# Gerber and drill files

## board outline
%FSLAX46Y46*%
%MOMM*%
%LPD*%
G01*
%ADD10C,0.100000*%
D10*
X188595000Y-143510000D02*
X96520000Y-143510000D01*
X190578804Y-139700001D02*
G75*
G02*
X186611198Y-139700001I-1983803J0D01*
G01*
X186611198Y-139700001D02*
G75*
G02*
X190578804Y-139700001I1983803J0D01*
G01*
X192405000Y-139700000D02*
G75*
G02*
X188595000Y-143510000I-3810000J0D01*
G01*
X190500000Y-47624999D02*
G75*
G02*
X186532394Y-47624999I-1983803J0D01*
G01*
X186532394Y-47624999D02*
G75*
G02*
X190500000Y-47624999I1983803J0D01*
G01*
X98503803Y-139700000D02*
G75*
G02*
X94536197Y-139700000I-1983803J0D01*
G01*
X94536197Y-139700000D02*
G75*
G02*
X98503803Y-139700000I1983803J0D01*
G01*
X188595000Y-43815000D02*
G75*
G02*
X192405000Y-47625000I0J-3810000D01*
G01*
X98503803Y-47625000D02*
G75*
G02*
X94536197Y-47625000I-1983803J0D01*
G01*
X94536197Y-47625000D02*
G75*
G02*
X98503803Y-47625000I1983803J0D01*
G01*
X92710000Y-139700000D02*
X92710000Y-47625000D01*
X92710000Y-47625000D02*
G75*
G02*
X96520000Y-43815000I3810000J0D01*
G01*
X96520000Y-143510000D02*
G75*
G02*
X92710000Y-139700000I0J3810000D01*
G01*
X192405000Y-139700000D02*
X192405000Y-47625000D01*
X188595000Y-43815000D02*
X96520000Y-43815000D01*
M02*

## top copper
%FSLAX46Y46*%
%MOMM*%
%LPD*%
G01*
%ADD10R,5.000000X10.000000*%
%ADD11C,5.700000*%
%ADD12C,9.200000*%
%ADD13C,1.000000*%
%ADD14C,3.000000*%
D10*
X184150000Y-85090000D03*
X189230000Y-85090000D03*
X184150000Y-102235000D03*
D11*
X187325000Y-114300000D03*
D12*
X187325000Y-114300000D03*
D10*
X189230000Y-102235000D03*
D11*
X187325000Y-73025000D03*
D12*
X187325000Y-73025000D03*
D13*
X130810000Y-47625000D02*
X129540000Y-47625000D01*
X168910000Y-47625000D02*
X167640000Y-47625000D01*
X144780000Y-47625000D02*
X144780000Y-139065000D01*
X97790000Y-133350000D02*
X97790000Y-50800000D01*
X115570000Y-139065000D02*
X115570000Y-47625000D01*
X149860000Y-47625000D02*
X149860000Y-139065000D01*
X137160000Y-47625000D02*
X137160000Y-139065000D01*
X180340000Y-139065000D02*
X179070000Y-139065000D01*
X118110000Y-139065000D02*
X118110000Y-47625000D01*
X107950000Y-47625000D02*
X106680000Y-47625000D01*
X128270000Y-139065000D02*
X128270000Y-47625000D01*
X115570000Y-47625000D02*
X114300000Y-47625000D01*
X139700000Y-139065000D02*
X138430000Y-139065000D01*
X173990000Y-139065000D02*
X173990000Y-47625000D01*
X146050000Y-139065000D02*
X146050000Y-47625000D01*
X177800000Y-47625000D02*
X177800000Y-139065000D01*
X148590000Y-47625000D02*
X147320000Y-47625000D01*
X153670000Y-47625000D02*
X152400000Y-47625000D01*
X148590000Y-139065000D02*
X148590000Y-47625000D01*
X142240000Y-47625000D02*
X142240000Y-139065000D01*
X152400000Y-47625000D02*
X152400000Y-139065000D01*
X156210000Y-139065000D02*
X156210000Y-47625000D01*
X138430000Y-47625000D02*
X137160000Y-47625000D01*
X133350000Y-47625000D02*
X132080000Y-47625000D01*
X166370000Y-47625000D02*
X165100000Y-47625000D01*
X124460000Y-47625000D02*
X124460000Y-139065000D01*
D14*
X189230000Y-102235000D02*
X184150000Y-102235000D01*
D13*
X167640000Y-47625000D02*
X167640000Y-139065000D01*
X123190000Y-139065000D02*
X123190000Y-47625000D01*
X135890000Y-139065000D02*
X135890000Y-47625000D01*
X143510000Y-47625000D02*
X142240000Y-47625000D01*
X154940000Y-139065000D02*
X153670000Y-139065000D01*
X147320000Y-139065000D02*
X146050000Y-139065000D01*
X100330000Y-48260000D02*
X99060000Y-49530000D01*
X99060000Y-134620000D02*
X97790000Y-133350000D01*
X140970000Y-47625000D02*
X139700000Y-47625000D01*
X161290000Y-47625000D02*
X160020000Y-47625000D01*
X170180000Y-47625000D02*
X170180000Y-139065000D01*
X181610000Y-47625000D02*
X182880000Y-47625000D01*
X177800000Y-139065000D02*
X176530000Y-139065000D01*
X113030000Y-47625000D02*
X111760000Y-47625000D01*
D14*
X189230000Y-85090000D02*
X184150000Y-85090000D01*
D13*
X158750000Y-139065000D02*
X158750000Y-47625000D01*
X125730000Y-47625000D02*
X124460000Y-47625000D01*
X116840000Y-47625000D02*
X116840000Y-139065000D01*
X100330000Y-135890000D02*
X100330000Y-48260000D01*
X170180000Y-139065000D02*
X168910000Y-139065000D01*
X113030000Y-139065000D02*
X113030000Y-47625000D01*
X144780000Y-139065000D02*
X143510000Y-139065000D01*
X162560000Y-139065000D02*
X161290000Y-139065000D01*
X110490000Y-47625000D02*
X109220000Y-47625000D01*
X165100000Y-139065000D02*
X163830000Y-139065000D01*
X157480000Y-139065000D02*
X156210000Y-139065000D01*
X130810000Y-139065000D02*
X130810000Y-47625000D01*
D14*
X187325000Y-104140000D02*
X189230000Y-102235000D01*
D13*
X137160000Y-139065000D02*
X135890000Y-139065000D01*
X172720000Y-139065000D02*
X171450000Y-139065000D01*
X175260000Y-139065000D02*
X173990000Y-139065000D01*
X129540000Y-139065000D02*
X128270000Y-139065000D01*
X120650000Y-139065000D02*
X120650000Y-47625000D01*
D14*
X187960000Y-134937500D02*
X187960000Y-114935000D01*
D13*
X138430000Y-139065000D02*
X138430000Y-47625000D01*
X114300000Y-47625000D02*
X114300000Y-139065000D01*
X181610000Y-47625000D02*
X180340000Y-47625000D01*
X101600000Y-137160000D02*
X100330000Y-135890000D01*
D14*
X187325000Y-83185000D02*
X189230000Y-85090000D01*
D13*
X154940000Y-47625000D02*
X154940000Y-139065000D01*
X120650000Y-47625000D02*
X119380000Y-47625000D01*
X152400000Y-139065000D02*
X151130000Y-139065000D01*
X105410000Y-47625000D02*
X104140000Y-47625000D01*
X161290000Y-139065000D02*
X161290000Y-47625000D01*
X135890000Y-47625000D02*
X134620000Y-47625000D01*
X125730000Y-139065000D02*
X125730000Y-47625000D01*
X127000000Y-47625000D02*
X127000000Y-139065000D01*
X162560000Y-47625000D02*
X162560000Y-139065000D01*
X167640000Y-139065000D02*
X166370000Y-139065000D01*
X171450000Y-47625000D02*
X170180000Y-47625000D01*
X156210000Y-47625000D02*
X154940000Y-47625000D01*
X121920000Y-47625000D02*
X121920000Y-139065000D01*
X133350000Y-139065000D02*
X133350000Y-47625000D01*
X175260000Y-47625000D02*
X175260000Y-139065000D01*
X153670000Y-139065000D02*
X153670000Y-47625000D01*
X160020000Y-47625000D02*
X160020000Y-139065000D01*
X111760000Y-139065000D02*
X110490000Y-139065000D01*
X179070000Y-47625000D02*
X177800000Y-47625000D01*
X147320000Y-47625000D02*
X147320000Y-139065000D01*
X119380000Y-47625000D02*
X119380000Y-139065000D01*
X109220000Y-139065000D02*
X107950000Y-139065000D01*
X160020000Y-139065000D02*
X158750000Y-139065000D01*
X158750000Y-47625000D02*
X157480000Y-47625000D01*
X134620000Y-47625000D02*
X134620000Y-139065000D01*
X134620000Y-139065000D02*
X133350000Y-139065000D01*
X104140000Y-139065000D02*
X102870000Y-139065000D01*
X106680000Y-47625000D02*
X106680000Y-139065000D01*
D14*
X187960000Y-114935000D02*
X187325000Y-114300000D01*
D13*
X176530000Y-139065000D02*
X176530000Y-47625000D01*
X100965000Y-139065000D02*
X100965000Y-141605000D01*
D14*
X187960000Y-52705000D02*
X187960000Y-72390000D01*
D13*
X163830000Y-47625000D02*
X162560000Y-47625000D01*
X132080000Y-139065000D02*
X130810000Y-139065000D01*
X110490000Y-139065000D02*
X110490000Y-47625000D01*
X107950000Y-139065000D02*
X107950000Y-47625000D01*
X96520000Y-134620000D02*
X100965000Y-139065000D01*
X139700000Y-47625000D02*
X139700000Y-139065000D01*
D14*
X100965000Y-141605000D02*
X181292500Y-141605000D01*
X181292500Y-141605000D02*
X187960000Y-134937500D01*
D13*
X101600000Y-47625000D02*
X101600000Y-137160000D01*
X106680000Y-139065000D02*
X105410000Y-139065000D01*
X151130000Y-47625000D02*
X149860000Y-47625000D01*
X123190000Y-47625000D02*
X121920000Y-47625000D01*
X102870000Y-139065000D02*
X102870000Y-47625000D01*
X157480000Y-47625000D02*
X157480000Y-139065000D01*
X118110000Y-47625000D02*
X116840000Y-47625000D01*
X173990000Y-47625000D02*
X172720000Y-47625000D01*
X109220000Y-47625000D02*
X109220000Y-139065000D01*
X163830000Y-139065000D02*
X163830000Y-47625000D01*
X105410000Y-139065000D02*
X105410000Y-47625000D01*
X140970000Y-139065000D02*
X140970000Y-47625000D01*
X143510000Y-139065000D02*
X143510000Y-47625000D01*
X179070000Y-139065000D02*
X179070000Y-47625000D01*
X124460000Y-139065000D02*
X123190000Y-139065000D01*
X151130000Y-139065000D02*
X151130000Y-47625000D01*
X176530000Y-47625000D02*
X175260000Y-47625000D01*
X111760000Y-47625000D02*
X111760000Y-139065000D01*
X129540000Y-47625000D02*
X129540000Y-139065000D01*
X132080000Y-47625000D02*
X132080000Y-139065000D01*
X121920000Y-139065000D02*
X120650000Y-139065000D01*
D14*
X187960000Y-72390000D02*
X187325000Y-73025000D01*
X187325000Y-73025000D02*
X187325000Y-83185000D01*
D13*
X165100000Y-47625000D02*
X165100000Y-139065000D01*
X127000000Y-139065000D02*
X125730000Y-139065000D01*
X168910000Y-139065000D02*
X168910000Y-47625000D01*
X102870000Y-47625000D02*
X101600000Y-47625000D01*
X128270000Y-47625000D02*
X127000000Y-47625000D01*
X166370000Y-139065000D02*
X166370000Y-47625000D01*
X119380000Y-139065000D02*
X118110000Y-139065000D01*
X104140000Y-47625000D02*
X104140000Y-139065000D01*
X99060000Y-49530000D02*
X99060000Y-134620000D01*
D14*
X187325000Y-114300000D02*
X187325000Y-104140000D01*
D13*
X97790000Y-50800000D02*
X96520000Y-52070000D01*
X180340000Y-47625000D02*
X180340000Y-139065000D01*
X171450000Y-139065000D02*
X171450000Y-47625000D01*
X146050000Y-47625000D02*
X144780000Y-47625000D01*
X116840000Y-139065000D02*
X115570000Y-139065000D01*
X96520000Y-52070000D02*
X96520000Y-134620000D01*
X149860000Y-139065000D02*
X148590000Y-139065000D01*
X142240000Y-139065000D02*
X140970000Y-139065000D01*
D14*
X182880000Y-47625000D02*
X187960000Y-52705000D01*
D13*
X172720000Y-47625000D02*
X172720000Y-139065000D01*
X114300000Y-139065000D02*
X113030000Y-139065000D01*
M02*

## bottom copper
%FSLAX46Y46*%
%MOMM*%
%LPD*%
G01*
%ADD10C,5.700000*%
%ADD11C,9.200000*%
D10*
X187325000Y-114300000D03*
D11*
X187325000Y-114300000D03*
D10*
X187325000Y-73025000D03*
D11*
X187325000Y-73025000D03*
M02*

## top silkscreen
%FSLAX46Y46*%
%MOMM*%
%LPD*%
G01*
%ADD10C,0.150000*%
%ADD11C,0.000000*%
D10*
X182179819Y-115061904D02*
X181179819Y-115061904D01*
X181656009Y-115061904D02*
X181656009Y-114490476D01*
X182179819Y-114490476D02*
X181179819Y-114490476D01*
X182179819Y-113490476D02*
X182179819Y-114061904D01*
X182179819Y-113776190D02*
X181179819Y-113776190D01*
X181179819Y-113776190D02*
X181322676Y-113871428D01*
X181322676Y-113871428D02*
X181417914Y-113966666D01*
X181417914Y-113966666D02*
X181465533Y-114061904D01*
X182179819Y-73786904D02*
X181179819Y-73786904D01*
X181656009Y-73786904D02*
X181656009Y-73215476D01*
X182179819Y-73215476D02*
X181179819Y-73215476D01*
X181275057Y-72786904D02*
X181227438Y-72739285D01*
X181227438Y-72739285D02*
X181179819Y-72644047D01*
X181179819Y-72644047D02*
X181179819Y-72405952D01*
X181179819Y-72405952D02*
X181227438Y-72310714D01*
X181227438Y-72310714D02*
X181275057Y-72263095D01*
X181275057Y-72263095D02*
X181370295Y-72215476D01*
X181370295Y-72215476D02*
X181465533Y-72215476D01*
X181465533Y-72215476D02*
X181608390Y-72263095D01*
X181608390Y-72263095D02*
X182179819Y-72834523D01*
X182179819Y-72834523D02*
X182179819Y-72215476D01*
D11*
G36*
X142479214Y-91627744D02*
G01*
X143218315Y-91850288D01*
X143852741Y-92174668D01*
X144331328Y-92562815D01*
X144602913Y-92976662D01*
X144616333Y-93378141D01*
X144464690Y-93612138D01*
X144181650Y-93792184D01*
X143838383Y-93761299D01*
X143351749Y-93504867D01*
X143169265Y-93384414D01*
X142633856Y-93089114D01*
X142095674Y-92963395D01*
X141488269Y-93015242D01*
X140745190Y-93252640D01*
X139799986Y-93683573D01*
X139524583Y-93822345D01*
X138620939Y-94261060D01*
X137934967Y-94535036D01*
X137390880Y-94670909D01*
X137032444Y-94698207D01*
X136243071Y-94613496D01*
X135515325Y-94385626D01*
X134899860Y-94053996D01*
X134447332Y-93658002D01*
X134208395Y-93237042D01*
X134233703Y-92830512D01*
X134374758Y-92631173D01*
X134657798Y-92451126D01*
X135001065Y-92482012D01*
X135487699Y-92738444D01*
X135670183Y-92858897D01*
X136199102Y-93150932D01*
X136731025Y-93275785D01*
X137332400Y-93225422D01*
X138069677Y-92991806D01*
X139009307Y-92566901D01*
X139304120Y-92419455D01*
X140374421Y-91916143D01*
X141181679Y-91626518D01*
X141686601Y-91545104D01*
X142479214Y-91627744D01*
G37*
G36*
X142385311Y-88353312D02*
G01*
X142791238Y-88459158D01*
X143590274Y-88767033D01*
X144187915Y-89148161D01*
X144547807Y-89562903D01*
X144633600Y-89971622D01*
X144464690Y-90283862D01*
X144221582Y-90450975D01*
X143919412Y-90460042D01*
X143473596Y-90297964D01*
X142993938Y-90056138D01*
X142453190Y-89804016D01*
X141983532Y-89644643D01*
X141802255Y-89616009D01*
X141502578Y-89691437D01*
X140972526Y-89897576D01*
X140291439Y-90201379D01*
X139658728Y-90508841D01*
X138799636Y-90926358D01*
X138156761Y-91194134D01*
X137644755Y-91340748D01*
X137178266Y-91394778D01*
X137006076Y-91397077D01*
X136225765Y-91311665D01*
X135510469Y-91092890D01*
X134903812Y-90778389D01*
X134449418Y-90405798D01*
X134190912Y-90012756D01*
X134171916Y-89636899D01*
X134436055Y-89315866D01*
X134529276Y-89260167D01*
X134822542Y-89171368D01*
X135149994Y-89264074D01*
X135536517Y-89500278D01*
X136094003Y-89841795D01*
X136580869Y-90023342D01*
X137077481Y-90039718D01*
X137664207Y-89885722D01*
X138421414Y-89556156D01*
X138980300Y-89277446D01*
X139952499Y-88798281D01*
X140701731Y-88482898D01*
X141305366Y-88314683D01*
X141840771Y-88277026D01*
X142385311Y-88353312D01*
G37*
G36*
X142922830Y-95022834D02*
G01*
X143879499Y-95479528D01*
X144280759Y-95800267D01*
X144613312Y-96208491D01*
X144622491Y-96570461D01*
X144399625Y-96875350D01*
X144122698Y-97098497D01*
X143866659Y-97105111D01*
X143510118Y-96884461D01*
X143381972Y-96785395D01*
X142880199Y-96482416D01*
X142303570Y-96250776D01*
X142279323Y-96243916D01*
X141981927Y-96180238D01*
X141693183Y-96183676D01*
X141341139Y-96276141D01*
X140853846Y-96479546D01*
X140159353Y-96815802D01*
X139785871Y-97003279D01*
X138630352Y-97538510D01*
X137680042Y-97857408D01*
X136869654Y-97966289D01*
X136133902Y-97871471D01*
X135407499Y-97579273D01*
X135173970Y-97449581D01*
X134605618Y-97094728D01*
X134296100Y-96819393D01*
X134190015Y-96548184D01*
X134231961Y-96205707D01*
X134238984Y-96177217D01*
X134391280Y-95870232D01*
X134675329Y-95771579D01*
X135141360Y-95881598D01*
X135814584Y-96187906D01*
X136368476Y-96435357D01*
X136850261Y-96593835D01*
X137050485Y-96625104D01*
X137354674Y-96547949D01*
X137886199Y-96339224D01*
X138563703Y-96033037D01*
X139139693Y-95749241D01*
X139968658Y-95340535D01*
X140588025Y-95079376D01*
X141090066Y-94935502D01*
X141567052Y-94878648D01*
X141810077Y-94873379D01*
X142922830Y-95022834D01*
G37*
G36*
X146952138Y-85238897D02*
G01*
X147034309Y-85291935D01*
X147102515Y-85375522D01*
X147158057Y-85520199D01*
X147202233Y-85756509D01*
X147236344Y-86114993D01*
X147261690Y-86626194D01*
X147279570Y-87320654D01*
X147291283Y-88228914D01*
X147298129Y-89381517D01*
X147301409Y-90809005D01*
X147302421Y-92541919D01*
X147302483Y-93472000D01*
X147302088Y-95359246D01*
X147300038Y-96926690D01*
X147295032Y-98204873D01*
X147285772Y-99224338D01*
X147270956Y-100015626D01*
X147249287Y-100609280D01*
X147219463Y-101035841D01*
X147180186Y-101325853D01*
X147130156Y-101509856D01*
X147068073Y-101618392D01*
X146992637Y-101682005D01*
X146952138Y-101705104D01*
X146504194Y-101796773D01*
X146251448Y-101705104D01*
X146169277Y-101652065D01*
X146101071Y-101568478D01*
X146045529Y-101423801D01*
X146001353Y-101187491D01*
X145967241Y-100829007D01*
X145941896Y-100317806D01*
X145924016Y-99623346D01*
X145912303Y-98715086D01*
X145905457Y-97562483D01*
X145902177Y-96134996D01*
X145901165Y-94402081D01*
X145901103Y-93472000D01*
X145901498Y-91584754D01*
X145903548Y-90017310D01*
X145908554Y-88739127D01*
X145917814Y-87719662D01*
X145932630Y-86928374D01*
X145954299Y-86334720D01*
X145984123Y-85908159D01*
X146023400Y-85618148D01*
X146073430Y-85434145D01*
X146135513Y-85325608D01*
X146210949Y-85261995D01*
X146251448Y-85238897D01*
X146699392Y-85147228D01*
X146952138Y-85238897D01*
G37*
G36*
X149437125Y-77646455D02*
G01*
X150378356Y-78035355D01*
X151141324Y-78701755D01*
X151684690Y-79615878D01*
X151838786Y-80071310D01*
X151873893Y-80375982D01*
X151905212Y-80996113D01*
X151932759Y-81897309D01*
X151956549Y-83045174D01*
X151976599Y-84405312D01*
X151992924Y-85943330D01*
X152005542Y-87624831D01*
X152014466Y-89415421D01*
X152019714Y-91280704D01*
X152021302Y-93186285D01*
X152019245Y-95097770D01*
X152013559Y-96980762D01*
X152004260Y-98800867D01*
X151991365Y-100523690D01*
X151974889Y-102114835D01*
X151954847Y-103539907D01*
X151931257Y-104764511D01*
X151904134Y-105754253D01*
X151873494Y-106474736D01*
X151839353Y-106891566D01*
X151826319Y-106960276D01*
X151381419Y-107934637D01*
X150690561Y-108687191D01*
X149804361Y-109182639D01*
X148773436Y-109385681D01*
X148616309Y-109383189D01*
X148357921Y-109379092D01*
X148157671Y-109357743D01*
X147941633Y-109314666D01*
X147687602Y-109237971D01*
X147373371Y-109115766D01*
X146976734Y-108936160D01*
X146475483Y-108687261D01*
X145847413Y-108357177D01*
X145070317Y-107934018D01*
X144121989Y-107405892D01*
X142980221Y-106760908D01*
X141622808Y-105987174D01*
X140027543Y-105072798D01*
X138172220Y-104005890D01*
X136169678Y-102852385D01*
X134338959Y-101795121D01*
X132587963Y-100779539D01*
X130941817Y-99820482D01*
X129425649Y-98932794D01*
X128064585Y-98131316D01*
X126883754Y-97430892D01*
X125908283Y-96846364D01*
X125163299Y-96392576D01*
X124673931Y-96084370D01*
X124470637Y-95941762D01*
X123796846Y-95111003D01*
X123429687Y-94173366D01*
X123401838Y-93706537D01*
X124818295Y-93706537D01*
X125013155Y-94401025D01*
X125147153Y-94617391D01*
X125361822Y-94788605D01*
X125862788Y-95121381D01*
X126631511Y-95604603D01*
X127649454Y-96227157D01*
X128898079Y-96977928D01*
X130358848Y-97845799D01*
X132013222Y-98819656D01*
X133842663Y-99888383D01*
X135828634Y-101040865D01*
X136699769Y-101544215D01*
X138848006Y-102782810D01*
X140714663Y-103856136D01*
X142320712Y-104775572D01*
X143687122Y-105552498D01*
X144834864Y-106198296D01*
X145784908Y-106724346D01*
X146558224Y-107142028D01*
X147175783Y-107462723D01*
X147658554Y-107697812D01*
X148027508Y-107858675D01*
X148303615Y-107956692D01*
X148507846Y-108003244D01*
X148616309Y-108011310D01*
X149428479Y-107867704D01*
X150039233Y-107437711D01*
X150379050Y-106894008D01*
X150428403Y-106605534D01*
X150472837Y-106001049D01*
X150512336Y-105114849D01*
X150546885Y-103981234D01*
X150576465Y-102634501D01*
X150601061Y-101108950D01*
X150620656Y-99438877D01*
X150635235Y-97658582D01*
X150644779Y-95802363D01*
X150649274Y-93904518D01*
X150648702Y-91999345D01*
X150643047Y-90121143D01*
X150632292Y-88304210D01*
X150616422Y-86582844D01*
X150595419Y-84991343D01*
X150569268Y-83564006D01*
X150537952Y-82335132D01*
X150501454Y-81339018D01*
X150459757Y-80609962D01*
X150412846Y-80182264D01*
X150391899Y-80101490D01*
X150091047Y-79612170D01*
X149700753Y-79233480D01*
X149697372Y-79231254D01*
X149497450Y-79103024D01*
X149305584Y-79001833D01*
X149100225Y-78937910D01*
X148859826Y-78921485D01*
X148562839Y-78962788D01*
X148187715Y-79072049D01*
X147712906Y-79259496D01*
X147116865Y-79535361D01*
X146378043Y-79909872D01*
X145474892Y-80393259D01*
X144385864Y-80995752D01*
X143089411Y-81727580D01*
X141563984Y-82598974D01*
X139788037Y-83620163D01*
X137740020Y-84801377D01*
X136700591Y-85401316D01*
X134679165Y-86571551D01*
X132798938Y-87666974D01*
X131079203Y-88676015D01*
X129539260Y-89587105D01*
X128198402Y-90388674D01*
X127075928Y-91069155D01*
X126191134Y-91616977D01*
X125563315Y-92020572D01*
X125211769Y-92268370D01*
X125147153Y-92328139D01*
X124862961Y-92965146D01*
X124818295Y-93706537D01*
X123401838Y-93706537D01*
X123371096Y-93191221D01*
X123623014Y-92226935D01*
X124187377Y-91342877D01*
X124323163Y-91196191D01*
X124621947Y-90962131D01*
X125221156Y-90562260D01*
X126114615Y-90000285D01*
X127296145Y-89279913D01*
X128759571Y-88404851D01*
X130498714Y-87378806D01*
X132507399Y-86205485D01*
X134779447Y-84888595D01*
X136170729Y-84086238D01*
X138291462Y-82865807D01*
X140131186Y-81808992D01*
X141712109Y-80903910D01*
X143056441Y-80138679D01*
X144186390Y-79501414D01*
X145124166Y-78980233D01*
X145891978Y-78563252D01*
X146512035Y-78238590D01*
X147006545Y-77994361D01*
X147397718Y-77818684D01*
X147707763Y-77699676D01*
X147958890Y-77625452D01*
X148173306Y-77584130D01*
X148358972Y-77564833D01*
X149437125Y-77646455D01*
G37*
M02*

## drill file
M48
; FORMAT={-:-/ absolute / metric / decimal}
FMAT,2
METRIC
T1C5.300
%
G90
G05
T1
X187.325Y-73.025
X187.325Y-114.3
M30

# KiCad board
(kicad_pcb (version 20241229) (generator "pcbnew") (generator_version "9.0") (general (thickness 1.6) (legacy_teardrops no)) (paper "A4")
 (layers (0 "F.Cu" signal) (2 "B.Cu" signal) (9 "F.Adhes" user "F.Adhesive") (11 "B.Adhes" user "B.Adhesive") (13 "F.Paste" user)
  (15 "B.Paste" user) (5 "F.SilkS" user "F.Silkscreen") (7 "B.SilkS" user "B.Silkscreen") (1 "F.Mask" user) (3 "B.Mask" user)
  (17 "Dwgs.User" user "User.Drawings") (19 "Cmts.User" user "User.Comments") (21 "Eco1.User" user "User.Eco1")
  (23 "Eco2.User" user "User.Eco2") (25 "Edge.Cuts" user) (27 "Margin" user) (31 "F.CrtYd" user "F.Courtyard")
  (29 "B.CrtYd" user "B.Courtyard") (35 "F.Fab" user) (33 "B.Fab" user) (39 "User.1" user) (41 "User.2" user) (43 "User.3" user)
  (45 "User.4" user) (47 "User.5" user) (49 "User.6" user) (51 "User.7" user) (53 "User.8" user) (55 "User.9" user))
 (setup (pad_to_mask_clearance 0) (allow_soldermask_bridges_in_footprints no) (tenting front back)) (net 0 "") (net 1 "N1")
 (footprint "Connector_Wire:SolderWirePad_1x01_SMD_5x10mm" (layer "F.Cu") (at 184.15 85.09)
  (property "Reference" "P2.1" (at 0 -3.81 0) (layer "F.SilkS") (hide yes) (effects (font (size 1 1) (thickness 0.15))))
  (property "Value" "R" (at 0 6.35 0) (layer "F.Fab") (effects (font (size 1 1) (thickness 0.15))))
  (pad "1" smd rect (at 0 0) (size 5 10) (layers "F.Cu" "F.Mask" "F.Paste") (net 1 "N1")))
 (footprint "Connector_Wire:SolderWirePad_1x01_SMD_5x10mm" (layer "F.Cu") (at 189.23 85.09)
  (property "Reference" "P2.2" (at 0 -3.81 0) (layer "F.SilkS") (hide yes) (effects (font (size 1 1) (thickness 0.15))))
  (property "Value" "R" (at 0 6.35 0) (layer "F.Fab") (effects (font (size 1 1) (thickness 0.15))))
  (pad "1" smd rect (at 0 0) (size 5 10) (layers "F.Cu" "F.Mask" "F.Paste") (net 1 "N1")))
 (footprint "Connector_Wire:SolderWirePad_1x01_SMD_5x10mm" (layer "F.Cu") (at 184.15 102.235)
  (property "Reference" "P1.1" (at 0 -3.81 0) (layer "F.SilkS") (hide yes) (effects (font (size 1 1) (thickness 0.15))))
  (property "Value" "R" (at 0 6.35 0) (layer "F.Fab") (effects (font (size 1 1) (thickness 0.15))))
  (pad "1" smd rect (at 0 0) (size 5 10) (layers "F.Cu" "F.Mask" "F.Paste") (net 1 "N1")))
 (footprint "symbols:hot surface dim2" (layer "F.Cu") (at 137.668 93.472 90)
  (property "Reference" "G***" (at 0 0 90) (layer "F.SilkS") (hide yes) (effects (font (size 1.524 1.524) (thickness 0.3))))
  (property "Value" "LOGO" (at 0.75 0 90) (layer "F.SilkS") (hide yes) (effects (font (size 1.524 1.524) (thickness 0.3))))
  (fp_poly
   (pts (xy 0.641488 -3.434297) (xy 0.840827 -3.293242) (xy 1.020874 -3.010202) (xy 0.989988 -2.666935) (xy 0.733556 -2.180301)
    (xy 0.613103 -1.997817) (xy 0.321068 -1.468898) (xy 0.196215 -0.936975) (xy 0.246578 -0.3356) (xy 0.480194 0.401677)
    (xy 0.905099 1.341307) (xy 1.052545 1.63612) (xy 1.555857 2.706421) (xy 1.845482 3.513679) (xy 1.926896 4.018601) (xy 1.844256 4.811214)
    (xy 1.621712 5.550315) (xy 1.297332 6.184741) (xy 0.909185 6.663328) (xy 0.495338 6.934913) (xy 0.093859 6.948333)
    (xy -0.140138 6.79669) (xy -0.320184 6.51365) (xy -0.289299 6.170383) (xy -0.032867 5.683749) (xy 0.087586 5.501265)
    (xy 0.382886 4.965856) (xy 0.508605 4.427674) (xy 0.456758 3.820269) (xy 0.21936 3.07719) (xy -0.211573 2.131986)
    (xy -0.350345 1.856583) (xy -0.78906 0.952939) (xy -1.063036 0.266967) (xy -1.198909 -0.27712) (xy -1.226207 -0.635556)
    (xy -1.141496 -1.424929) (xy -0.913626 -2.152675) (xy -0.581996 -2.76814) (xy -0.186002 -3.220668) (xy 0.234958 -3.459605))
   (stroke (width 0) (type solid)) (fill yes) (layer "F.SilkS"))
  (fp_poly
   (pts (xy 4.156134 -3.231945) (xy 4.211833 -3.138724) (xy 4.300632 -2.845458) (xy 4.207926 -2.518006) (xy 3.971722 -2.131483)
    (xy 3.630205 -1.573997) (xy 3.448658 -1.087131) (xy 3.432282 -0.590519) (xy 3.586278 -0.003793) (xy 3.915844 0.753414)
    (xy 4.194554 1.3123) (xy 4.673719 2.284499) (xy 4.989102 3.033731) (xy 5.157317 3.637366) (xy 5.194974 4.172771) (xy 5.118688 4.717311)
    (xy 5.012842 5.123238) (xy 4.704967 5.922274) (xy 4.323839 6.519915) (xy 3.909097 6.879807) (xy 3.500378 6.9656) (xy 3.188138 6.79669)
    (xy 3.021025 6.553582) (xy 3.011958 6.251412) (xy 3.174036 5.805596) (xy 3.415862 5.325938) (xy 3.667984 4.78519) (xy 3.827357 4.315532)
    (xy 3.855991 4.134255) (xy 3.780563 3.834578) (xy 3.574424 3.304526) (xy 3.270621 2.623439) (xy 2.963159 1.990728)
    (xy 2.545642 1.131636) (xy 2.277866 0.488761) (xy 2.131252 -0.023245) (xy 2.077222 -0.489734) (xy 2.074923 -0.661924)
    (xy 2.160335 -1.442235) (xy 2.37911 -2.157531) (xy 2.693611 -2.764188) (xy 3.066202 -3.218582) (xy 3.459244 -3.477088)
    (xy 3.835101 -3.496084))
   (stroke (width 0) (type solid)) (fill yes) (layer "F.SilkS"))
  (fp_poly
   (pts (xy -2.733707 -3.436039) (xy -2.705217 -3.429016) (xy -2.398232 -3.27672) (xy -2.299579 -2.992671) (xy -2.409598 -2.52664)
    (xy -2.715906 -1.853416) (xy -2.963357 -1.299524) (xy -3.121835 -0.817739) (xy -3.153104 -0.617515) (xy -3.075949 -0.313326)
    (xy -2.867224 0.218199) (xy -2.561037 0.895703) (xy -2.277241 1.471693) (xy -1.868535 2.300658) (xy -1.607376 2.920025)
    (xy -1.463502 3.422066) (xy -1.406648 3.899052) (xy -1.401379 4.142077) (xy -1.550834 5.25483) (xy -2.007528 6.211499)
    (xy -2.328267 6.612759) (xy -2.736491 6.945312) (xy -3.098461 6.954491) (xy -3.40335 6.731625) (xy -3.626497 6.454698)
    (xy -3.633111 6.198659) (xy -3.412461 5.842118) (xy -3.313395 5.713972) (xy -3.010416 5.212199) (xy -2.778776 4.63557)
    (xy -2.771916 4.611323) (xy -2.708238 4.313927) (xy -2.711676 4.025183) (xy -2.804141 3.673139) (xy -3.007546 3.185846)
    (xy -3.343802 2.491353) (xy -3.531279 2.117871) (xy -4.06651 0.962352) (xy -4.385408 0.012042) (xy -4.494289 -0.798346)
    (xy -4.399471 -1.534098) (xy -4.107273 -2.260501) (xy -3.977581 -2.49403) (xy -3.622728 -3.062382) (xy -3.347393 -3.3719)
    (xy -3.076184 -3.477985))
   (stroke (width 0) (type solid)) (fill yes) (layer "F.SilkS"))
  (fp_poly
   (pts (xy 1.887246 8.233498) (xy 3.45469 8.235548) (xy 4.732873 8.240554) (xy 5.752338 8.249814) (xy 6.543626 8.26463)
    (xy 7.13728 8.286299) (xy 7.563841 8.316123) (xy 7.853852 8.3554) (xy 8.037855 8.40543) (xy 8.146392 8.467513) (xy 8.210005 8.542949)
    (xy 8.233103 8.583448) (xy 8.324772 9.031392) (xy 8.233103 9.284138) (xy 8.180065 9.366309) (xy 8.096478 9.434515)
    (xy 7.951801 9.490057) (xy 7.715491 9.534233) (xy 7.357007 9.568344) (xy 6.845806 9.59369) (xy 6.151346 9.61157) (xy 5.243086 9.623283)
    (xy 4.090483 9.630129) (xy 2.662995 9.633409) (xy 0.930081 9.634421) (xy 0 9.634483) (xy -1.887246 9.634088) (xy -3.45469 9.632038)
    (xy -4.732873 9.627032) (xy -5.752338 9.617772) (xy -6.543626 9.602956) (xy -7.13728 9.581287) (xy -7.563841 9.551463)
    (xy -7.853853 9.512186) (xy -8.037856 9.462156) (xy -8.146392 9.400073) (xy -8.210005 9.324637) (xy -8.233104 9.284138)
    (xy -8.324773 8.836194) (xy -8.233104 8.583448) (xy -8.180065 8.501277) (xy -8.096478 8.433071) (xy -7.951801 8.377529)
    (xy -7.715491 8.333353) (xy -7.357007 8.299241) (xy -6.845806 8.273896) (xy -6.151346 8.256016) (xy -5.243086 8.244303)
    (xy -4.090483 8.237457) (xy -2.662996 8.234177) (xy -0.930081 8.233165) (xy 0 8.233103))
   (stroke (width 0) (type solid)) (fill yes) (layer "F.SilkS"))
  (fp_poly
   (pts (xy 1.245065 -14.044986) (xy 2.129123 -13.480623) (xy 2.275809 -13.344837) (xy 2.509869 -13.046053) (xy 2.90974 -12.446844)
    (xy 3.471715 -11.553385) (xy 4.192087 -10.371855) (xy 5.067149 -8.908429) (xy 6.093194 -7.169286) (xy 7.266515 -5.160601)
    (xy 8.583405 -2.888553) (xy 9.385762 -1.497271) (xy 10.606193 0.623462) (xy 11.663008 2.463186) (xy 12.56809 4.044109)
    (xy 13.333321 5.388441) (xy 13.970586 6.51839) (xy 14.491767 7.456166) (xy 14.908748 8.223978) (xy 15.23341 8.844035)
    (xy 15.477639 9.338545) (xy 15.653316 9.729718) (xy 15.772324 10.039763) (xy 15.846548 10.29089) (xy 15.88787 10.505306)
    (xy 15.907167 10.690972) (xy 15.825545 11.769125) (xy 15.436645 12.710356) (xy 14.770245 13.473324) (xy 13.856122 14.01669)
    (xy 13.40069 14.170786) (xy 13.096018 14.205893) (xy 12.475887 14.237212) (xy 11.574691 14.264759) (xy 10.426826 14.288549)
    (xy 9.066688 14.308599) (xy 7.52867 14.324924) (xy 5.847169 14.337542) (xy 4.056579 14.346466) (xy 2.191296 14.351714)
    (xy 0.285715 14.353302) (xy -1.62577 14.351245) (xy -3.508762 14.345559) (xy -5.328867 14.33626) (xy -7.05169 14.323365)
    (xy -8.642835 14.306889) (xy -10.067907 14.286847) (xy -11.292511 14.263257) (xy -12.282253 14.236134) (xy -13.002736 14.205494)
    (xy -13.419566 14.171353) (xy -13.488276 14.158319) (xy -14.462637 13.713419) (xy -15.215191 13.022561) (xy -15.710639 12.136361)
    (xy -15.913681 11.105436) (xy -15.911189 10.948309) (xy -14.53931 10.948309) (xy -14.395704 11.760479) (xy -13.965711 12.371233)
    (xy -13.422008 12.71105) (xy -13.133534 12.760403) (xy -12.529049 12.804837) (xy -11.642849 12.844336) (xy -10.509234 12.878885)
    (xy -9.162501 12.908465) (xy -7.63695 12.933061) (xy -5.966877 12.952656) (xy -4.186582 12.967235) (xy -2.330363 12.976779)
    (xy -0.432518 12.981274) (xy 1.472655 12.980702) (xy 3.350857 12.975047) (xy 5.16779 12.964292) (xy 6.889156 12.948422)
    (xy 8.480657 12.927419) (xy 9.907994 12.901268) (xy 11.136868 12.869952) (xy 12.132982 12.833454) (xy 12.862038 12.791757)
    (xy 13.289736 12.744846) (xy 13.37051 12.723899) (xy 13.85983 12.423047) (xy 14.23852 12.032753) (xy 14.240746 12.029372)
    (xy 14.368976 11.82945) (xy 14.470167 11.637584) (xy 14.53409 11.432225) (xy 14.550515 11.191826) (xy 14.509212 10.894839)
    (xy 14.399951 10.519715) (xy 14.212504 10.044906) (xy 13.936639 9.448865) (xy 13.562128 8.710043) (xy 13.078741 7.806892)
    (xy 12.476248 6.717864) (xy 11.74442 5.421411) (xy 10.873026 3.895984) (xy 9.851837 2.120037) (xy 8.670623 0.07202)
    (xy 8.070684 -0.967409) (xy 6.900449 -2.988835) (xy 5.805026 -4.869062) (xy 4.795985 -6.588797) (xy 3.884895 -8.12874)
    (xy 3.083326 -9.469598) (xy 2.402845 -10.592072) (xy 1.855023 -11.476866) (xy 1.451428 -12.104685) (xy 1.20363 -12.456231)
    (xy 1.143861 -12.520847) (xy 0.506854 -12.805039) (xy -0.234537 -12.849705) (xy -0.929025 -12.654845) (xy -1.145391 -12.520847)
    (xy -1.316605 -12.306178) (xy -1.649381 -11.805212) (xy -2.132603 -11.036489) (xy -2.755157 -10.018546) (xy -3.505928 -8.769921)
    (xy -4.373799 -7.309152) (xy -5.347656 -5.654778) (xy -6.416383 -3.825337) (xy -7.568865 -1.839366) (xy -8.072215 -0.968231)
    (xy -9.31081 1.180006) (xy -10.384136 3.046663) (xy -11.303572 4.652712) (xy -12.080498 6.019122) (xy -12.726296 7.166864)
    (xy -13.252346 8.116908) (xy -13.670028 8.890224) (xy -13.990723 9.507783) (xy -14.225812 9.990554) (xy -14.386675 10.359508)
    (xy -14.484692 10.635615) (xy -14.531244 10.839846) (xy -14.53931 10.948309) (xy -15.911189 10.948309) (xy -15.907092 10.689921)
    (xy -15.885743 10.489671) (xy -15.842666 10.273633) (xy -15.765971 10.019602) (xy -15.643766 9.705371) (xy -15.46416 9.308734)
    (xy -15.215261 8.807483) (xy -14.885177 8.179413) (xy -14.462018 7.402317) (xy -13.933892 6.453989) (xy -13.288908 5.312221)
    (xy -12.515174 3.954808) (xy -11.600798 2.359543) (xy -10.53389 0.50422) (xy -9.380385 -1.498322) (xy -8.323121 -3.329041)
    (xy -7.307539 -5.080037) (xy -6.348482 -6.726183) (xy -5.460794 -8.242351) (xy -4.659316 -9.603415) (xy -3.958892 -10.784246)
    (xy -3.374364 -11.759717) (xy -2.920576 -12.504701) (xy -2.61237 -12.994069) (xy -2.469762 -13.197363) (xy -1.639003 -13.871154)
    (xy -0.701366 -14.238313) (xy 0.280779 -14.296904))
   (stroke (width 0) (type solid)) (fill yes) (layer "F.SilkS")))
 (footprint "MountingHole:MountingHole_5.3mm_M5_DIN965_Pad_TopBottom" (layer "F.Cu") (at 187.325 114.3 90)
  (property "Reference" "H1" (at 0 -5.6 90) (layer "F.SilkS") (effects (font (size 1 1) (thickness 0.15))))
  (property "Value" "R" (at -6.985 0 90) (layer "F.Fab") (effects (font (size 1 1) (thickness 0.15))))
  (pad "1" thru_hole circle (at 0 0 90) (size 5.7 5.7) (drill 5.3) (layers "*.Cu" "*.Mask") (remove_unused_layers no) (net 1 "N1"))
  (pad "1" connect circle (at 0 0 90) (size 9.2 9.2) (layers "F.Cu" "F.Mask") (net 1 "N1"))
  (pad "1" connect circle (at 0 0 90) (size 9.2 9.2) (layers "B.Cu" "B.Mask") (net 1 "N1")))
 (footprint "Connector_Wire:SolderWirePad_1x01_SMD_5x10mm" (layer "F.Cu") (at 189.23 102.235)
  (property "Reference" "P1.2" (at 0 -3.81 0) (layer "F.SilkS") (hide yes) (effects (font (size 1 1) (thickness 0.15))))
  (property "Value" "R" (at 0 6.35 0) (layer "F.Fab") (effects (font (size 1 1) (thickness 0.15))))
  (pad "1" smd rect (at 0 0) (size 5 10) (layers "F.Cu" "F.Mask" "F.Paste") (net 1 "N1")))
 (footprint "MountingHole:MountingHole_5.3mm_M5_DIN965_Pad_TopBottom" (layer "F.Cu") (at 187.325 73.025 90)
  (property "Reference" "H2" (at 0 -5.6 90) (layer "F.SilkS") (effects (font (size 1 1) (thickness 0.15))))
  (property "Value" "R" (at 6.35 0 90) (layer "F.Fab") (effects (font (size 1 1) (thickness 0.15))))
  (pad "1" thru_hole circle (at 0 0 90) (size 5.7 5.7) (drill 5.3) (layers "*.Cu" "*.Mask") (remove_unused_layers no) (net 1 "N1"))
  (pad "1" connect circle (at 0 0 90) (size 9.2 9.2) (layers "F.Cu" "F.Mask") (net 1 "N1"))
  (pad "1" connect circle (at 0 0 90) (size 9.2 9.2) (layers "B.Cu" "B.Mask") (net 1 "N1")))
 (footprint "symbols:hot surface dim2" (layer "B.Cu") (at 137.668 93.472 -90)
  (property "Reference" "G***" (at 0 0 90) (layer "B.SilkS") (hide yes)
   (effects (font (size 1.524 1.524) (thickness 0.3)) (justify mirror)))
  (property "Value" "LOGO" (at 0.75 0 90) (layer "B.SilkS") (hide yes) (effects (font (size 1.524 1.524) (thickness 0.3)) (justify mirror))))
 (gr_line (start 188.595 143.51) (end 96.52 143.51) (stroke (width 0.1) (type solid)) (layer "Edge.Cuts"))
 (gr_circle (center 188.595001 139.700001) (end 187.071001 138.430001) (stroke (width 0.1) (type solid)) (fill no) (layer "Edge.Cuts"))
 (gr_arc (start 192.405 139.7) (mid 191.289077 142.394077) (end 188.595 143.51) (stroke (width 0.1) (type solid)) (layer "Edge.Cuts"))
 (gr_circle (center 188.516197 47.624999) (end 186.992197 46.354999) (stroke (width 0.1) (type solid)) (fill no) (layer "Edge.Cuts"))
 (gr_circle (center 96.52 139.7) (end 94.996 138.43) (stroke (width 0.1) (type solid)) (fill no) (layer "Edge.Cuts"))
 (gr_arc (start 188.595 43.815) (mid 191.289077 44.930923) (end 192.405 47.625) (stroke (width 0.1) (type solid)) (layer "Edge.Cuts"))
 (gr_circle (center 96.52 47.625) (end 94.996 46.355) (stroke (width 0.1) (type solid)) (fill no) (layer "Edge.Cuts"))
 (gr_line (start 92.71 139.7) (end 92.71 47.625) (stroke (width 0.1) (type solid)) (layer "Edge.Cuts"))
 (gr_arc (start 92.71 47.625) (mid 93.825923 44.930923) (end 96.52 43.815) (stroke (width 0.1) (type solid)) (layer "Edge.Cuts"))
 (gr_arc (start 96.52 143.51) (mid 93.825923 142.394077) (end 92.71 139.7) (stroke (width 0.1) (type solid)) (layer "Edge.Cuts"))
 (gr_line (start 192.405 139.7) (end 192.405 47.625) (stroke (width 0.1) (type solid)) (layer "Edge.Cuts"))
 (gr_line (start 188.595 43.815) (end 96.52 43.815) (stroke (width 0.1) (type solid)) (layer "Edge.Cuts"))
 (segment (start 130.81 47.625) (end 129.54 47.625) (width 1) (layer "F.Cu") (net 1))
 (segment (start 168.91 47.625) (end 167.64 47.625) (width 1) (layer "F.Cu") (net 1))
 (segment (start 144.78 47.625) (end 144.78 139.065) (width 1) (layer "F.Cu") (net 1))
 (segment (start 97.79 133.35) (end 97.79 50.8) (width 1) (layer "F.Cu") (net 1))
 (segment (start 115.57 139.065) (end 115.57 47.625) (width 1) (layer "F.Cu") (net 1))
 (segment (start 149.86 47.625) (end 149.86 139.065) (width 1) (layer "F.Cu") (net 1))
 (segment (start 137.16 47.625) (end 137.16 139.065) (width 1) (layer "F.Cu") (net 1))
 (segment (start 180.34 139.065) (end 179.07 139.065) (width 1) (layer "F.Cu") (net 1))
 (segment (start 118.11 139.065) (end 118.11 47.625) (width 1) (layer "F.Cu") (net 1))
 (segment (start 107.95 47.625) (end 106.68 47.625) (width 1) (layer "F.Cu") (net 1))
 (segment (start 128.27 139.065) (end 128.27 47.625) (width 1) (layer "F.Cu") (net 1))
 (segment (start 115.57 47.625) (end 114.3 47.625) (width 1) (layer "F.Cu") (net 1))
 (segment (start 139.7 139.065) (end 138.43 139.065) (width 1) (layer "F.Cu") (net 1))
 (segment (start 173.99 139.065) (end 173.99 47.625) (width 1) (layer "F.Cu") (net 1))
 (segment (start 146.05 139.065) (end 146.05 47.625) (width 1) (layer "F.Cu") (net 1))
 (segment (start 177.8 47.625) (end 177.8 139.065) (width 1) (layer "F.Cu") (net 1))
 (segment (start 148.59 47.625) (end 147.32 47.625) (width 1) (layer "F.Cu") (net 1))
 (segment (start 153.67 47.625) (end 152.4 47.625) (width 1) (layer "F.Cu") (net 1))
 (segment (start 148.59 139.065) (end 148.59 47.625) (width 1) (layer "F.Cu") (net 1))
 (segment (start 142.24 47.625) (end 142.24 139.065) (width 1) (layer "F.Cu") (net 1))
 (segment (start 152.4 47.625) (end 152.4 139.065) (width 1) (layer "F.Cu") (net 1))
 (segment (start 156.21 139.065) (end 156.21 47.625) (width 1) (layer "F.Cu") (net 1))
 (segment (start 138.43 47.625) (end 137.16 47.625) (width 1) (layer "F.Cu") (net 1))
 (segment (start 133.35 47.625) (end 132.08 47.625) (width 1) (layer "F.Cu") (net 1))
 (segment (start 166.37 47.625) (end 165.1 47.625) (width 1) (layer "F.Cu") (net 1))
 (segment (start 124.46 47.625) (end 124.46 139.065) (width 1) (layer "F.Cu") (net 1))
 (segment (start 189.23 102.235) (end 184.15 102.235) (width 3) (layer "F.Cu") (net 1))
 (segment (start 167.64 47.625) (end 167.64 139.065) (width 1) (layer "F.Cu") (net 1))
 (segment (start 123.19 139.065) (end 123.19 47.625) (width 1) (layer "F.Cu") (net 1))
 (segment (start 135.89 139.065) (end 135.89 47.625) (width 1) (layer "F.Cu") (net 1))
 (segment (start 143.51 47.625) (end 142.24 47.625) (width 1) (layer "F.Cu") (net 1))
 (segment (start 154.94 139.065) (end 153.67 139.065) (width 1) (layer "F.Cu") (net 1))
 (segment (start 147.32 139.065) (end 146.05 139.065) (width 1) (layer "F.Cu") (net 1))
 (segment (start 100.33 48.26) (end 99.06 49.53) (width 1) (layer "F.Cu") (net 1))
 (segment (start 99.06 134.62) (end 97.79 133.35) (width 1) (layer "F.Cu") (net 1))
 (segment (start 140.97 47.625) (end 139.7 47.625) (width 1) (layer "F.Cu") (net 1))
 (segment (start 161.29 47.625) (end 160.02 47.625) (width 1) (layer "F.Cu") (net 1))
 (segment (start 170.18 47.625) (end 170.18 139.065) (width 1) (layer "F.Cu") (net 1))
 (segment (start 181.61 47.625) (end 182.88 47.625) (width 1) (layer "F.Cu") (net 1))
 (segment (start 177.8 139.065) (end 176.53 139.065) (width 1) (layer "F.Cu") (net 1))
 (segment (start 113.03 47.625) (end 111.76 47.625) (width 1) (layer "F.Cu") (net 1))
 (segment (start 189.23 85.09) (end 184.15 85.09) (width 3) (layer "F.Cu") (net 1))
 (segment (start 158.75 139.065) (end 158.75 47.625) (width 1) (layer "F.Cu") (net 1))
 (segment (start 125.73 47.625) (end 124.46 47.625) (width 1) (layer "F.Cu") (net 1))
 (segment (start 116.84 47.625) (end 116.84 139.065) (width 1) (layer "F.Cu") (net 1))
 (segment (start 100.33 135.89) (end 100.33 48.26) (width 1) (layer "F.Cu") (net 1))
 (segment (start 170.18 139.065) (end 168.91 139.065) (width 1) (layer "F.Cu") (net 1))
 (segment (start 113.03 139.065) (end 113.03 47.625) (width 1) (layer "F.Cu") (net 1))
 (segment (start 144.78 139.065) (end 143.51 139.065) (width 1) (layer "F.Cu") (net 1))
 (segment (start 162.56 139.065) (end 161.29 139.065) (width 1) (layer "F.Cu") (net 1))
 (segment (start 110.49 47.625) (end 109.22 47.625) (width 1) (layer "F.Cu") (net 1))
 (segment (start 165.1 139.065) (end 163.83 139.065) (width 1) (layer "F.Cu") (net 1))
 (segment (start 157.48 139.065) (end 156.21 139.065) (width 1) (layer "F.Cu") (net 1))
 (segment (start 130.81 139.065) (end 130.81 47.625) (width 1) (layer "F.Cu") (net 1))
 (segment (start 187.325 104.14) (end 189.23 102.235) (width 3) (layer "F.Cu") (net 1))
 (segment (start 137.16 139.065) (end 135.89 139.065) (width 1) (layer "F.Cu") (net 1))
 (segment (start 172.72 139.065) (end 171.45 139.065) (width 1) (layer "F.Cu") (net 1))
 (segment (start 175.26 139.065) (end 173.99 139.065) (width 1) (layer "F.Cu") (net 1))
 (segment (start 129.54 139.065) (end 128.27 139.065) (width 1) (layer "F.Cu") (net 1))
 (segment (start 120.65 139.065) (end 120.65 47.625) (width 1) (layer "F.Cu") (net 1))
 (segment (start 187.96 134.9375) (end 187.96 114.935) (width 3) (layer "F.Cu") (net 1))
 (segment (start 138.43 139.065) (end 138.43 47.625) (width 1) (layer "F.Cu") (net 1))
 (segment (start 114.3 47.625) (end 114.3 139.065) (width 1) (layer "F.Cu") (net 1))
 (segment (start 181.61 47.625) (end 180.34 47.625) (width 1) (layer "F.Cu") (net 1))
 (segment (start 101.6 137.16) (end 100.33 135.89) (width 1) (layer "F.Cu") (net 1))
 (segment (start 187.325 83.185) (end 189.23 85.09) (width 3) (layer "F.Cu") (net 1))
 (segment (start 154.94 47.625) (end 154.94 139.065) (width 1) (layer "F.Cu") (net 1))
 (segment (start 120.65 47.625) (end 119.38 47.625) (width 1) (layer "F.Cu") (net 1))
 (segment (start 152.4 139.065) (end 151.13 139.065) (width 1) (layer "F.Cu") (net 1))
 (segment (start 105.41 47.625) (end 104.14 47.625) (width 1) (layer "F.Cu") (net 1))
 (segment (start 161.29 139.065) (end 161.29 47.625) (width 1) (layer "F.Cu") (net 1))
 (segment (start 135.89 47.625) (end 134.62 47.625) (width 1) (layer "F.Cu") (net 1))
 (segment (start 125.73 139.065) (end 125.73 47.625) (width 1) (layer "F.Cu") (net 1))
 (segment (start 127 47.625) (end 127 139.065) (width 1) (layer "F.Cu") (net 1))
 (segment (start 162.56 47.625) (end 162.56 139.065) (width 1) (layer "F.Cu") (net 1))
 (segment (start 167.64 139.065) (end 166.37 139.065) (width 1) (layer "F.Cu") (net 1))
 (segment (start 171.45 47.625) (end 170.18 47.625) (width 1) (layer "F.Cu") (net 1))
 (segment (start 156.21 47.625) (end 154.94 47.625) (width 1) (layer "F.Cu") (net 1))
 (segment (start 121.92 47.625) (end 121.92 139.065) (width 1) (layer "F.Cu") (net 1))
 (segment (start 133.35 139.065) (end 133.35 47.625) (width 1) (layer "F.Cu") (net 1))
 (segment (start 175.26 47.625) (end 175.26 139.065) (width 1) (layer "F.Cu") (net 1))
 (segment (start 153.67 139.065) (end 153.67 47.625) (width 1) (layer "F.Cu") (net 1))
 (segment (start 160.02 47.625) (end 160.02 139.065) (width 1) (layer "F.Cu") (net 1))
 (segment (start 111.76 139.065) (end 110.49 139.065) (width 1) (layer "F.Cu") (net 1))
 (segment (start 179.07 47.625) (end 177.8 47.625) (width 1) (layer "F.Cu") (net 1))
 (segment (start 147.32 47.625) (end 147.32 139.065) (width 1) (layer "F.Cu") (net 1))
 (segment (start 119.38 47.625) (end 119.38 139.065) (width 1) (layer "F.Cu") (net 1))
 (segment (start 109.22 139.065) (end 107.95 139.065) (width 1) (layer "F.Cu") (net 1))
 (segment (start 160.02 139.065) (end 158.75 139.065) (width 1) (layer "F.Cu") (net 1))
 (segment (start 158.75 47.625) (end 157.48 47.625) (width 1) (layer "F.Cu") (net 1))
 (segment (start 134.62 47.625) (end 134.62 139.065) (width 1) (layer "F.Cu") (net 1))
 (segment (start 134.62 139.065) (end 133.35 139.065) (width 1) (layer "F.Cu") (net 1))
 (segment (start 104.14 139.065) (end 102.87 139.065) (width 1) (layer "F.Cu") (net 1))
 (segment (start 106.68 47.625) (end 106.68 139.065) (width 1) (layer "F.Cu") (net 1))
 (segment (start 187.96 114.935) (end 187.325 114.3) (width 3) (layer "F.Cu") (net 1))
 (segment (start 176.53 139.065) (end 176.53 47.625) (width 1) (layer "F.Cu") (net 1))
 (segment (start 100.965 139.065) (end 100.965 141.605) (width 1) (layer "F.Cu") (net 1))
 (segment (start 187.96 52.705) (end 187.96 72.39) (width 3) (layer "F.Cu") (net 1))
 (segment (start 163.83 47.625) (end 162.56 47.625) (width 1) (layer "F.Cu") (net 1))
 (segment (start 132.08 139.065) (end 130.81 139.065) (width 1) (layer "F.Cu") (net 1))
 (segment (start 110.49 139.065) (end 110.49 47.625) (width 1) (layer "F.Cu") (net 1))
 (segment (start 107.95 139.065) (end 107.95 47.625) (width 1) (layer "F.Cu") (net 1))
 (segment (start 96.52 134.62) (end 100.965 139.065) (width 1) (layer "F.Cu") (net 1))
 (segment (start 139.7 47.625) (end 139.7 139.065) (width 1) (layer "F.Cu") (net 1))
 (segment (start 100.965 141.605) (end 181.2925 141.605) (width 3) (layer "F.Cu") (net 1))
 (segment (start 181.2925 141.605) (end 187.96 134.9375) (width 3) (layer "F.Cu") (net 1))
 (segment (start 101.6 47.625) (end 101.6 137.16) (width 1) (layer "F.Cu") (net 1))
 (segment (start 106.68 139.065) (end 105.41 139.065) (width 1) (layer "F.Cu") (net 1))
 (segment (start 151.13 47.625) (end 149.86 47.625) (width 1) (layer "F.Cu") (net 1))
 (segment (start 123.19 47.625) (end 121.92 47.625) (width 1) (layer "F.Cu") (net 1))
 (segment (start 102.87 139.065) (end 102.87 47.625) (width 1) (layer "F.Cu") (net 1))
 (segment (start 157.48 47.625) (end 157.48 139.065) (width 1) (layer "F.Cu") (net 1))
 (segment (start 118.11 47.625) (end 116.84 47.625) (width 1) (layer "F.Cu") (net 1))
 (segment (start 173.99 47.625) (end 172.72 47.625) (width 1) (layer "F.Cu") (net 1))
 (segment (start 109.22 47.625) (end 109.22 139.065) (width 1) (layer "F.Cu") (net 1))
 (segment (start 163.83 139.065) (end 163.83 47.625) (width 1) (layer "F.Cu") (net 1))
 (segment (start 105.41 139.065) (end 105.41 47.625) (width 1) (layer "F.Cu") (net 1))
 (segment (start 140.97 139.065) (end 140.97 47.625) (width 1) (layer "F.Cu") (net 1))
 (segment (start 143.51 139.065) (end 143.51 47.625) (width 1) (layer "F.Cu") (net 1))
 (segment (start 179.07 139.065) (end 179.07 47.625) (width 1) (layer "F.Cu") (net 1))
 (segment (start 124.46 139.065) (end 123.19 139.065) (width 1) (layer "F.Cu") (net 1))
 (segment (start 151.13 139.065) (end 151.13 47.625) (width 1) (layer "F.Cu") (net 1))
 (segment (start 176.53 47.625) (end 175.26 47.625) (width 1) (layer "F.Cu") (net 1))
 (segment (start 111.76 47.625) (end 111.76 139.065) (width 1) (layer "F.Cu") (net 1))
 (segment (start 129.54 47.625) (end 129.54 139.065) (width 1) (layer "F.Cu") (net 1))
 (segment (start 132.08 47.625) (end 132.08 139.065) (width 1) (layer "F.Cu") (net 1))
 (segment (start 121.92 139.065) (end 120.65 139.065) (width 1) (layer "F.Cu") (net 1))
 (segment (start 187.96 72.39) (end 187.325 73.025) (width 3) (layer "F.Cu") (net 1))
 (segment (start 187.325 73.025) (end 187.325 83.185) (width 3) (layer "F.Cu") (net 1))
 (segment (start 165.1 47.625) (end 165.1 139.065) (width 1) (layer "F.Cu") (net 1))
 (segment (start 127 139.065) (end 125.73 139.065) (width 1) (layer "F.Cu") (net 1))
 (segment (start 168.91 139.065) (end 168.91 47.625) (width 1) (layer "F.Cu") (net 1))
 (segment (start 102.87 47.625) (end 101.6 47.625) (width 1) (layer "F.Cu") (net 1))
 (segment (start 128.27 47.625) (end 127 47.625) (width 1) (layer "F.Cu") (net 1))
 (segment (start 166.37 139.065) (end 166.37 47.625) (width 1) (layer "F.Cu") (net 1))
 (segment (start 119.38 139.065) (end 118.11 139.065) (width 1) (layer "F.Cu") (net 1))
 (segment (start 104.14 47.625) (end 104.14 139.065) (width 1) (layer "F.Cu") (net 1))
 (segment (start 99.06 49.53) (end 99.06 134.62) (width 1) (layer "F.Cu") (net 1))
 (segment (start 187.325 114.3) (end 187.325 104.14) (width 3) (layer "F.Cu") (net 1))
 (segment (start 97.79 50.8) (end 96.52 52.07) (width 1) (layer "F.Cu") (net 1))
 (segment (start 180.34 47.625) (end 180.34 139.065) (width 1) (layer "F.Cu") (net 1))
 (segment (start 171.45 139.065) (end 171.45 47.625) (width 1) (layer "F.Cu") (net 1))
 (segment (start 146.05 47.625) (end 144.78 47.625) (width 1) (layer "F.Cu") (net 1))
 (segment (start 116.84 139.065) (end 115.57 139.065) (width 1) (layer "F.Cu") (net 1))
 (segment (start 96.52 52.07) (end 96.52 134.62) (width 1) (layer "F.Cu") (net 1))
 (segment (start 149.86 139.065) (end 148.59 139.065) (width 1) (layer "F.Cu") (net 1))
 (segment (start 142.24 139.065) (end 140.97 139.065) (width 1) (layer "F.Cu") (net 1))
 (segment (start 182.88 47.625) (end 187.96 52.705) (width 3) (layer "F.Cu") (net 1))
 (segment (start 172.72 47.625) (end 172.72 139.065) (width 1) (layer "F.Cu") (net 1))
 (segment (start 114.3 139.065) (end 113.03 139.065) (width 1) (layer "F.Cu") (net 1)))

